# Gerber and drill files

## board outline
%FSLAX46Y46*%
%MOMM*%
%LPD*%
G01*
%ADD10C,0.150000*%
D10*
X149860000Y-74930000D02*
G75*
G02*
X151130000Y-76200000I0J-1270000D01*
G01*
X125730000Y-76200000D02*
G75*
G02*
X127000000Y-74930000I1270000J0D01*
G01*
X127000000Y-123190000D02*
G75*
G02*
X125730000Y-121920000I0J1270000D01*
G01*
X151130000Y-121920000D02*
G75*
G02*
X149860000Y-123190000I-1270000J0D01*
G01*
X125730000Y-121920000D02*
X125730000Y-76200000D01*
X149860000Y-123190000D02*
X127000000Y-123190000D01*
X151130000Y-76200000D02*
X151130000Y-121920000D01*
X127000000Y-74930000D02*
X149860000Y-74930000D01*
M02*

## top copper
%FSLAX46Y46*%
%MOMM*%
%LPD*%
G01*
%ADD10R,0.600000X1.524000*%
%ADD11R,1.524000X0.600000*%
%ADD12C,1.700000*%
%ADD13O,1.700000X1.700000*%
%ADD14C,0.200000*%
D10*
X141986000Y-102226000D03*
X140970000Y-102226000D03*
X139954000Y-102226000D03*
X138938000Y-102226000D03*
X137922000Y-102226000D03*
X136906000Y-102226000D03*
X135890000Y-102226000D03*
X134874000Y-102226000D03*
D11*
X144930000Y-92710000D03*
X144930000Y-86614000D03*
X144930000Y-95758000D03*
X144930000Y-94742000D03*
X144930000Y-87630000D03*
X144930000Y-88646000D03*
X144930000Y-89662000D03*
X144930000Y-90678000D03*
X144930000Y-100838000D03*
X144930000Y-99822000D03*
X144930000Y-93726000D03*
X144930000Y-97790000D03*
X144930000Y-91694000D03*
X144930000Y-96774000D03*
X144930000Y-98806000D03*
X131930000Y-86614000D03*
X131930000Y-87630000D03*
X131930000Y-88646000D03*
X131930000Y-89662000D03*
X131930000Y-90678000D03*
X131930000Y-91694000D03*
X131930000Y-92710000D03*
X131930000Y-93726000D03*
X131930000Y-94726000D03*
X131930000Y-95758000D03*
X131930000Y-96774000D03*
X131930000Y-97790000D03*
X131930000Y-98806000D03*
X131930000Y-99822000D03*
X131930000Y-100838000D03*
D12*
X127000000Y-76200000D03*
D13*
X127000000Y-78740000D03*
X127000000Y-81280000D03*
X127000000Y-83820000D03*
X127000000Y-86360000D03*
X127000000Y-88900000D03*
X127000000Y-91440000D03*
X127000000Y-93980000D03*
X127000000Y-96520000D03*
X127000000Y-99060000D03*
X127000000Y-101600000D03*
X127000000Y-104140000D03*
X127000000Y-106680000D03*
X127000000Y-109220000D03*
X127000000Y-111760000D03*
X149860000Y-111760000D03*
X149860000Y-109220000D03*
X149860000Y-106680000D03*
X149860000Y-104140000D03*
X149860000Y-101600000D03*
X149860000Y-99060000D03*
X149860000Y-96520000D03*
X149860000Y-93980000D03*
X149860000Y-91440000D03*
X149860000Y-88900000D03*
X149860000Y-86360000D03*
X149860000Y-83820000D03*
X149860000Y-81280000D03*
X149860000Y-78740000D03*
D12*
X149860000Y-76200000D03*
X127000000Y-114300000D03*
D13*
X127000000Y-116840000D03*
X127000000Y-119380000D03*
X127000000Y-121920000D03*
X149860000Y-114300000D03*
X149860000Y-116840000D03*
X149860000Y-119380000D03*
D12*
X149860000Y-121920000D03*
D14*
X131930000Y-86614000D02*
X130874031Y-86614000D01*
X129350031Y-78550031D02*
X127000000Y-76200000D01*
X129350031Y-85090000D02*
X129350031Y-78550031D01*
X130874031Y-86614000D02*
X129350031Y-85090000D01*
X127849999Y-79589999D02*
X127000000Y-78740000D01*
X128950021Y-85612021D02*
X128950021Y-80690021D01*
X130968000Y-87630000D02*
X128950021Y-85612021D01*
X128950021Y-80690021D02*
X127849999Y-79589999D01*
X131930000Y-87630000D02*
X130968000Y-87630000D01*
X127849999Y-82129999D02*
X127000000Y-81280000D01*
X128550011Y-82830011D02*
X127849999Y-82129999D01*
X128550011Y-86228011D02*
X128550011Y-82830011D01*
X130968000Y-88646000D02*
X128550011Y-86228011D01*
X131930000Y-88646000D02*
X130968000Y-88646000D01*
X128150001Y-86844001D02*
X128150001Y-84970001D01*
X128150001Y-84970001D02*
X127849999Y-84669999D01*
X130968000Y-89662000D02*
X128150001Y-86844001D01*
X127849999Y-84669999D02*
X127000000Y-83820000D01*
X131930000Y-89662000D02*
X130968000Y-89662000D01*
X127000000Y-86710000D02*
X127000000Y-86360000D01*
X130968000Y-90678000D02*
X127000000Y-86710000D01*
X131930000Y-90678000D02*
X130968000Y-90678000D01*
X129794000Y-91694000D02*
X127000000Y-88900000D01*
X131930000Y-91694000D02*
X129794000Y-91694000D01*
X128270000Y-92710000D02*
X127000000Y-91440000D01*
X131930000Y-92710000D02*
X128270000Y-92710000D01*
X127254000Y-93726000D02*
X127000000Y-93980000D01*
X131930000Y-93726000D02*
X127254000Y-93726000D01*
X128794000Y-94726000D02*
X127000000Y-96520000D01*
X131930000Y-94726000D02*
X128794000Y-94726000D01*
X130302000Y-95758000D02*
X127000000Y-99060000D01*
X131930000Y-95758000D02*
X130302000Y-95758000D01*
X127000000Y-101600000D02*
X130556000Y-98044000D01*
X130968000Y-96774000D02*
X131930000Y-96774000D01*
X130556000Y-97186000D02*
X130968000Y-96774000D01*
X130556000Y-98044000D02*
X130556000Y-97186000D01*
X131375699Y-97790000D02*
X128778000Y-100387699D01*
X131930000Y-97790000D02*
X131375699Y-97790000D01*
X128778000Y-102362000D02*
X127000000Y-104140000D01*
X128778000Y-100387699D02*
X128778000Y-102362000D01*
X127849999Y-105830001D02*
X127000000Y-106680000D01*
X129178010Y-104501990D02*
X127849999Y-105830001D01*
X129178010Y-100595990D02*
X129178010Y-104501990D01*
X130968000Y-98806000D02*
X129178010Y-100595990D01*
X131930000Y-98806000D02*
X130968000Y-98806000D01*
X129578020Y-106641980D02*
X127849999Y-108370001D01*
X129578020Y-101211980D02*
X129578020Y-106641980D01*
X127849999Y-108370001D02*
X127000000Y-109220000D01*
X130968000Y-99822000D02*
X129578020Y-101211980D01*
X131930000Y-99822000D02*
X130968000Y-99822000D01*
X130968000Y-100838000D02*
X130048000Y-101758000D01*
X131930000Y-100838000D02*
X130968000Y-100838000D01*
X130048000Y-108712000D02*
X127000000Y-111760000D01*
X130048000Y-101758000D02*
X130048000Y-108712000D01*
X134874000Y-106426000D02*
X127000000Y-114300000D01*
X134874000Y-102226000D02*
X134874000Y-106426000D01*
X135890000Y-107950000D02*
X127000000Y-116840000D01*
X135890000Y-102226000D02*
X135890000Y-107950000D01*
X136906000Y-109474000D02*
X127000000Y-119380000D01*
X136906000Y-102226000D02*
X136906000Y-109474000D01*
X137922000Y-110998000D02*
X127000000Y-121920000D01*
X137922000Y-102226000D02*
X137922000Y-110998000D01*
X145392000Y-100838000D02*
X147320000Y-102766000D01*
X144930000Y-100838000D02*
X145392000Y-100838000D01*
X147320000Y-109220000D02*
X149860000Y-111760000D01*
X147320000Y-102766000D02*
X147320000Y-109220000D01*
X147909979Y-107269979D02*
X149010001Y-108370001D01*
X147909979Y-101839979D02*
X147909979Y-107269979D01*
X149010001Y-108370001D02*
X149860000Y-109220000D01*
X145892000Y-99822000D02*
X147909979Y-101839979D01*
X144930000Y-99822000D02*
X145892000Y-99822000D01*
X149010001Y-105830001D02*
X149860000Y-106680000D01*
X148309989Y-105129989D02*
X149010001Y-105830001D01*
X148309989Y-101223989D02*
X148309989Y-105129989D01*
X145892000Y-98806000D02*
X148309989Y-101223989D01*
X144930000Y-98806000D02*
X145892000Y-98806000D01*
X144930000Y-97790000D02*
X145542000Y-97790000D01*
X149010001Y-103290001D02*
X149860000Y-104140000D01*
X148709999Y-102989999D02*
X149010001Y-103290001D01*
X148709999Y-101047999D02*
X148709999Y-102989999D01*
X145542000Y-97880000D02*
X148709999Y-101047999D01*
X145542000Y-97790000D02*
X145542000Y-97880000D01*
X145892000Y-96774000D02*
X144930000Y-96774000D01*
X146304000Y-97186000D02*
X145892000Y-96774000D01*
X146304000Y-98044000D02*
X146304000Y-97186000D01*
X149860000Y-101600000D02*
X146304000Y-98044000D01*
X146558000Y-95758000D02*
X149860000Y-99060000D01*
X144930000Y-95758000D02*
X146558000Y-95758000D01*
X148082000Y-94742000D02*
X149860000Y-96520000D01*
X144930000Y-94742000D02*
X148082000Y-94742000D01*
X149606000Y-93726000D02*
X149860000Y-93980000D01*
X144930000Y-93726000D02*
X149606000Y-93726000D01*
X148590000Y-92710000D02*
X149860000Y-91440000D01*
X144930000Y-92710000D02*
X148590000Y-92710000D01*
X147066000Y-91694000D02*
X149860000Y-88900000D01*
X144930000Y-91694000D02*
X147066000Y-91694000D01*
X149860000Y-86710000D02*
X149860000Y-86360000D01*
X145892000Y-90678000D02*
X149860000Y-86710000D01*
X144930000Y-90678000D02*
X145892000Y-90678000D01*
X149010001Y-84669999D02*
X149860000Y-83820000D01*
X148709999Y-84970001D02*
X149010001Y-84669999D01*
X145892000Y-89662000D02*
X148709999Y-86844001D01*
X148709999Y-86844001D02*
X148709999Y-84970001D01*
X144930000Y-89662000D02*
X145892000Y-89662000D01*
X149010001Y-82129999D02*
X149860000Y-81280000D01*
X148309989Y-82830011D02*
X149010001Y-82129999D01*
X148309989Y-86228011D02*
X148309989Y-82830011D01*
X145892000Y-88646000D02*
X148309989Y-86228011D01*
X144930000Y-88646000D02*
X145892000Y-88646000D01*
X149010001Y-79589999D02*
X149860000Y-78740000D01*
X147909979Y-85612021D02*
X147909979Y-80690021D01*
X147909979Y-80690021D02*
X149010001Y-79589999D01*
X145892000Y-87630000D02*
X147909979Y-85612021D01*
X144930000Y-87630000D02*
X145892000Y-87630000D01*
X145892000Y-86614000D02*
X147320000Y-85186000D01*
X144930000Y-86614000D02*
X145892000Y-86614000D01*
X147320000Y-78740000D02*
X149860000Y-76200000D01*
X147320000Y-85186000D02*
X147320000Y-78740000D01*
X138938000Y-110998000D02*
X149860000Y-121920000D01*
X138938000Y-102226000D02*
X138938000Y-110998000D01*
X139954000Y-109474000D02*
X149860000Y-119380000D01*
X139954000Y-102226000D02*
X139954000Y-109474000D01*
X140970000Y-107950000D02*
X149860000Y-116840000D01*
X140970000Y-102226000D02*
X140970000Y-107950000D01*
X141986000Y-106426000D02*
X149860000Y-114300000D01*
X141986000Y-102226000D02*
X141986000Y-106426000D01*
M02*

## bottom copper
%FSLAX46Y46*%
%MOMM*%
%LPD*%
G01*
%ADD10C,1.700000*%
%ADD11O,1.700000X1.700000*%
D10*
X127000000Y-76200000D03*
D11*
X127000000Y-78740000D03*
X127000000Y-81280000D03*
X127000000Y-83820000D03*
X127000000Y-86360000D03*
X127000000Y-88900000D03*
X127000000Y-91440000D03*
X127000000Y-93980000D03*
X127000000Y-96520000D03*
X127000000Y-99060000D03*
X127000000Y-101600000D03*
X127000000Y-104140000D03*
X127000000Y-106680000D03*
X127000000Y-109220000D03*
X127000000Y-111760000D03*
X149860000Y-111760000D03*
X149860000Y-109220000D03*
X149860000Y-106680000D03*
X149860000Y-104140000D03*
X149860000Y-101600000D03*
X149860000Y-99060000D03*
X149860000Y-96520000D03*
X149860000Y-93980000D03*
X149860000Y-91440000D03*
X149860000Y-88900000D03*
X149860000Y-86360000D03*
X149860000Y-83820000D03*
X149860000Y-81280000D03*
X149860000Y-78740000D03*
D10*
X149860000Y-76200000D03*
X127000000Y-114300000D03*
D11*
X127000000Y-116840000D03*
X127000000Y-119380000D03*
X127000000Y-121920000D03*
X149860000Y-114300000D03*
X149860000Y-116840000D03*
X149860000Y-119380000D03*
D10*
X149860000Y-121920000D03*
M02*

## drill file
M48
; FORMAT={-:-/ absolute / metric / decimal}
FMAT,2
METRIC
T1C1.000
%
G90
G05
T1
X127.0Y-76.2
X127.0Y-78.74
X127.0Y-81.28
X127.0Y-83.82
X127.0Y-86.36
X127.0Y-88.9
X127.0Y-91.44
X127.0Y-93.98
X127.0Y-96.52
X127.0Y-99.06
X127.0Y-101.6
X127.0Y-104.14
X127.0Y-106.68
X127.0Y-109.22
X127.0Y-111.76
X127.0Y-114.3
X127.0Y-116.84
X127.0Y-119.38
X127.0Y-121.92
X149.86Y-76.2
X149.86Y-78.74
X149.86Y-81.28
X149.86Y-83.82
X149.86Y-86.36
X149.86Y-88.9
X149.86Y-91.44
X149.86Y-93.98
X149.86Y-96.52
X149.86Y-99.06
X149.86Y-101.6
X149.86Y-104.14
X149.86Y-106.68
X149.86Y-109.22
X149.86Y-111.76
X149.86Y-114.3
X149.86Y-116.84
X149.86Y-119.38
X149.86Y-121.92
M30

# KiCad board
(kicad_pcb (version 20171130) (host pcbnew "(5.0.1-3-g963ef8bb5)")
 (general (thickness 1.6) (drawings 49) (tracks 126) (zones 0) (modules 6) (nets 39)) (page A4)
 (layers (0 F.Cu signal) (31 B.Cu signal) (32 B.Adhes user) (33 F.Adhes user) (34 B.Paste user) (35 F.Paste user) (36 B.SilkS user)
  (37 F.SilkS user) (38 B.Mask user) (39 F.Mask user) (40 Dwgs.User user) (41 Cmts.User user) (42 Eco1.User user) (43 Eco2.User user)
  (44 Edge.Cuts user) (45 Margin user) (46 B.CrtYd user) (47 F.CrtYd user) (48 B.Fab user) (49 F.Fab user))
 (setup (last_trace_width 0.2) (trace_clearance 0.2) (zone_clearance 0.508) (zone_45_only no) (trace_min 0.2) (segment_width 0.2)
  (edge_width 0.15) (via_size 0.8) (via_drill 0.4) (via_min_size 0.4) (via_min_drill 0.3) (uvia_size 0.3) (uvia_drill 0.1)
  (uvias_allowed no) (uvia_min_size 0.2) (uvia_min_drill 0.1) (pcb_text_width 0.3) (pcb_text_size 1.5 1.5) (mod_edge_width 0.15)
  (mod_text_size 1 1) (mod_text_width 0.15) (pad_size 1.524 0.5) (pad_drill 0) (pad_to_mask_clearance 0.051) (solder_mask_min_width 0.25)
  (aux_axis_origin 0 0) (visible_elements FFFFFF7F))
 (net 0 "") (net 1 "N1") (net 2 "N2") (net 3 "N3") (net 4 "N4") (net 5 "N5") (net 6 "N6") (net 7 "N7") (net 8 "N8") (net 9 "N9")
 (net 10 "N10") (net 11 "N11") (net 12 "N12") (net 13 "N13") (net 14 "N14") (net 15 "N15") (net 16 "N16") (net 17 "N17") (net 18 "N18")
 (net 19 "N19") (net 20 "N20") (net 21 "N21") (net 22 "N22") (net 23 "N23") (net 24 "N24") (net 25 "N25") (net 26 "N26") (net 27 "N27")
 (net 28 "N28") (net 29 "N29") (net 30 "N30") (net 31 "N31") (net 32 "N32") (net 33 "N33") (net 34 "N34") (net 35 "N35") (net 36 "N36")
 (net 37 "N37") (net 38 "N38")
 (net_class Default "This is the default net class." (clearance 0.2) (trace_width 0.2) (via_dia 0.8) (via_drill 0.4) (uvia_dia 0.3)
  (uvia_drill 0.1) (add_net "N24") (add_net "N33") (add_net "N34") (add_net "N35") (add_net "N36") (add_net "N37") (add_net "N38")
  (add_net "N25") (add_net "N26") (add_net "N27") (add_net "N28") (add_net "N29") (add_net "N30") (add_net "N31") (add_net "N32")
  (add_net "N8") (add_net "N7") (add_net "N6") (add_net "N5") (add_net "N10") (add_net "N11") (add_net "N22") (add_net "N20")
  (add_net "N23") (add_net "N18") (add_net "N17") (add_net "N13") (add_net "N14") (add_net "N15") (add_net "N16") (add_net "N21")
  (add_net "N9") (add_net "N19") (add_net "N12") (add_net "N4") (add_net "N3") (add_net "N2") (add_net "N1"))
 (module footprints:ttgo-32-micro (layer F.Cu) (at 138.43 93.726)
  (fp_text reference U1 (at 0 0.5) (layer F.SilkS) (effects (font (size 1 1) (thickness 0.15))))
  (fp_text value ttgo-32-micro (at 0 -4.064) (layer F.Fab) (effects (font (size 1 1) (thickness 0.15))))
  (pad 23 smd rect (at 3.556 8.5 90) (size 1.524 0.6) (layers F.Cu F.Paste F.Mask) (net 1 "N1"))
  (pad 22 smd rect (at 2.54 8.5 90) (size 1.524 0.6) (layers F.Cu F.Paste F.Mask) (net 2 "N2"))
  (pad 21 smd rect (at 1.524 8.5 90) (size 1.524 0.6) (layers F.Cu F.Paste F.Mask) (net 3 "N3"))
  (pad 20 smd rect (at 0.508 8.5 90) (size 1.524 0.6) (layers F.Cu F.Paste F.Mask) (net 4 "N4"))
  (pad 19 smd rect (at -0.508 8.5 90) (size 1.524 0.6) (layers F.Cu F.Paste F.Mask) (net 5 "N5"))
  (pad 18 smd rect (at -1.524 8.5 90) (size 1.524 0.6) (layers F.Cu F.Paste F.Mask) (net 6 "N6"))
  (pad 17 smd rect (at -2.54 8.5 90) (size 1.524 0.6) (layers F.Cu F.Paste F.Mask) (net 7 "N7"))
  (pad 16 smd rect (at -3.556 8.5 90) (size 1.524 0.6) (layers F.Cu F.Paste F.Mask) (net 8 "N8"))
  (pad 32 smd rect (at 6.5 -1.016) (size 1.524 0.6) (layers F.Cu F.Paste F.Mask) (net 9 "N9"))
  (pad 38 smd rect (at 6.5 -7.112) (size 1.524 0.6) (layers F.Cu F.Paste F.Mask) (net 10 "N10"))
  (pad 29 smd rect (at 6.5 2.032) (size 1.524 0.6) (layers F.Cu F.Paste F.Mask) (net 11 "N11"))
  (pad 30 smd rect (at 6.5 1.016) (size 1.524 0.6) (layers F.Cu F.Paste F.Mask) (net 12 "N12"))
  (pad 37 smd rect (at 6.5 -6.096) (size 1.524 0.6) (layers F.Cu F.Paste F.Mask) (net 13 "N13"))
  (pad 36 smd rect (at 6.5 -5.08) (size 1.524 0.6) (layers F.Cu F.Paste F.Mask) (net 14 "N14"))
  (pad 35 smd rect (at 6.5 -4.064) (size 1.524 0.6) (layers F.Cu F.Paste F.Mask) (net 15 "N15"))
  (pad 34 smd rect (at 6.5 -3.048) (size 1.524 0.6) (layers F.Cu F.Paste F.Mask) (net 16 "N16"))
  (pad 24 smd rect (at 6.5 7.112) (size 1.524 0.6) (layers F.Cu F.Paste F.Mask) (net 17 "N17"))
  (pad 25 smd rect (at 6.5 6.096) (size 1.524 0.6) (layers F.Cu F.Paste F.Mask) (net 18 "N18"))
  (pad 31 smd rect (at 6.5 0) (size 1.524 0.6) (layers F.Cu F.Paste F.Mask) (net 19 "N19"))
  (pad 27 smd rect (at 6.5 4.064) (size 1.524 0.6) (layers F.Cu F.Paste F.Mask) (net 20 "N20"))
  (pad 33 smd rect (at 6.5 -2.032) (size 1.524 0.6) (layers F.Cu F.Paste F.Mask) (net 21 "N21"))
  (pad 28 smd rect (at 6.5 3.048) (size 1.524 0.6) (layers F.Cu F.Paste F.Mask) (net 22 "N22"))
  (pad 26 smd rect (at 6.5 5.08) (size 1.524 0.6) (layers F.Cu F.Paste F.Mask) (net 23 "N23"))
  (pad 1 smd rect (at -6.5 -7.112) (size 1.524 0.6) (layers F.Cu F.Paste F.Mask) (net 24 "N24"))
  (pad 2 smd rect (at -6.5 -6.096) (size 1.524 0.6) (layers F.Cu F.Paste F.Mask) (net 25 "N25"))
  (pad 3 smd rect (at -6.5 -5.08) (size 1.524 0.6) (layers F.Cu F.Paste F.Mask) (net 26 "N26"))
  (pad 4 smd rect (at -6.5 -4.064) (size 1.524 0.6) (layers F.Cu F.Paste F.Mask) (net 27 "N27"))
  (pad 5 smd rect (at -6.5 -3.048) (size 1.524 0.6) (layers F.Cu F.Paste F.Mask) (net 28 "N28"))
  (pad 6 smd rect (at -6.5 -2.032) (size 1.524 0.6) (layers F.Cu F.Paste F.Mask) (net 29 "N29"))
  (pad 7 smd rect (at -6.5 -1.016) (size 1.524 0.6) (layers F.Cu F.Paste F.Mask) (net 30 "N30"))
  (pad 8 smd rect (at -6.5 0) (size 1.524 0.6) (layers F.Cu F.Paste F.Mask) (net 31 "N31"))
  (pad 9 smd rect (at -6.5 1) (size 1.524 0.6) (layers F.Cu F.Paste F.Mask) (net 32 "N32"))
  (pad 10 smd rect (at -6.5 2.032) (size 1.524 0.6) (layers F.Cu F.Paste F.Mask) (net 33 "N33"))
  (pad 11 smd rect (at -6.5 3.048) (size 1.524 0.6) (layers F.Cu F.Paste F.Mask) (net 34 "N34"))
  (pad 12 smd rect (at -6.5 4.064) (size 1.524 0.6) (layers F.Cu F.Paste F.Mask) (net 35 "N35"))
  (pad 13 smd rect (at -6.5 5.08) (size 1.524 0.6) (layers F.Cu F.Paste F.Mask) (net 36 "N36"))
  (pad 14 smd rect (at -6.5 6.096) (size 1.524 0.6) (layers F.Cu F.Paste F.Mask) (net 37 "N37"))
  (pad 15 smd rect (at -6.5 7.112) (size 1.524 0.6) (layers F.Cu F.Paste F.Mask) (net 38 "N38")))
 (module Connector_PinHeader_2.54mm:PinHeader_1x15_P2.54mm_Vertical (layer B.Cu) (at 127 76.2 180)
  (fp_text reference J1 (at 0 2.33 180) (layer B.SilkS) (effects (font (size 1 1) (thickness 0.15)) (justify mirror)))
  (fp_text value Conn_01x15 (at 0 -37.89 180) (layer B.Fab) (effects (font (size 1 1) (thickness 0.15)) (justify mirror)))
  (pad 1 thru_hole circle (at 0 0 180) (size 1.7 1.7) (drill 1) (layers *.Cu *.Mask) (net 24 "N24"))
  (pad 2 thru_hole oval (at 0 -2.54 180) (size 1.7 1.7) (drill 1) (layers *.Cu *.Mask) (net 25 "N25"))
  (pad 3 thru_hole oval (at 0 -5.08 180) (size 1.7 1.7) (drill 1) (layers *.Cu *.Mask) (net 26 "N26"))
  (pad 4 thru_hole oval (at 0 -7.62 180) (size 1.7 1.7) (drill 1) (layers *.Cu *.Mask) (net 27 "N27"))
  (pad 5 thru_hole oval (at 0 -10.16 180) (size 1.7 1.7) (drill 1) (layers *.Cu *.Mask) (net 28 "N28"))
  (pad 6 thru_hole oval (at 0 -12.7 180) (size 1.7 1.7) (drill 1) (layers *.Cu *.Mask) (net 29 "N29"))
  (pad 7 thru_hole oval (at 0 -15.24 180) (size 1.7 1.7) (drill 1) (layers *.Cu *.Mask) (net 30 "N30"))
  (pad 8 thru_hole oval (at 0 -17.78 180) (size 1.7 1.7) (drill 1) (layers *.Cu *.Mask) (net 31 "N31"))
  (pad 9 thru_hole oval (at 0 -20.32 180) (size 1.7 1.7) (drill 1) (layers *.Cu *.Mask) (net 32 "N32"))
  (pad 10 thru_hole oval (at 0 -22.86 180) (size 1.7 1.7) (drill 1) (layers *.Cu *.Mask) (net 33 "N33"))
  (pad 11 thru_hole oval (at 0 -25.4 180) (size 1.7 1.7) (drill 1) (layers *.Cu *.Mask) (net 34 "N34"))
  (pad 12 thru_hole oval (at 0 -27.94 180) (size 1.7 1.7) (drill 1) (layers *.Cu *.Mask) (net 35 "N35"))
  (pad 13 thru_hole oval (at 0 -30.48 180) (size 1.7 1.7) (drill 1) (layers *.Cu *.Mask) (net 36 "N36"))
  (pad 14 thru_hole oval (at 0 -33.02 180) (size 1.7 1.7) (drill 1) (layers *.Cu *.Mask) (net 37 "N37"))
  (pad 15 thru_hole oval (at 0 -35.56 180) (size 1.7 1.7) (drill 1) (layers *.Cu *.Mask) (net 38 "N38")))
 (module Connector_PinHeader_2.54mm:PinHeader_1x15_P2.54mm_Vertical (layer B.Cu) (at 149.86 76.2 180)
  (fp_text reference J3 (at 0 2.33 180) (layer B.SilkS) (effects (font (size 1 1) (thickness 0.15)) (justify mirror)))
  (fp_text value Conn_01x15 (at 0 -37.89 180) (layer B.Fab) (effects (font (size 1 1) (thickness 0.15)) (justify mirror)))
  (pad 15 thru_hole oval (at 0 -35.56 180) (size 1.7 1.7) (drill 1) (layers *.Cu *.Mask) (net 17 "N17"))
  (pad 14 thru_hole oval (at 0 -33.02 180) (size 1.7 1.7) (drill 1) (layers *.Cu *.Mask) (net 18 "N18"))
  (pad 13 thru_hole oval (at 0 -30.48 180) (size 1.7 1.7) (drill 1) (layers *.Cu *.Mask) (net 23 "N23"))
  (pad 12 thru_hole oval (at 0 -27.94 180) (size 1.7 1.7) (drill 1) (layers *.Cu *.Mask) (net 20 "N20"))
  (pad 11 thru_hole oval (at 0 -25.4 180) (size 1.7 1.7) (drill 1) (layers *.Cu *.Mask) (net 22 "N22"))
  (pad 10 thru_hole oval (at 0 -22.86 180) (size 1.7 1.7) (drill 1) (layers *.Cu *.Mask) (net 11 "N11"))
  (pad 9 thru_hole oval (at 0 -20.32 180) (size 1.7 1.7) (drill 1) (layers *.Cu *.Mask) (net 12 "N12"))
  (pad 8 thru_hole oval (at 0 -17.78 180) (size 1.7 1.7) (drill 1) (layers *.Cu *.Mask) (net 19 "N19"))
  (pad 7 thru_hole oval (at 0 -15.24 180) (size 1.7 1.7) (drill 1) (layers *.Cu *.Mask) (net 9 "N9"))
  (pad 6 thru_hole oval (at 0 -12.7 180) (size 1.7 1.7) (drill 1) (layers *.Cu *.Mask) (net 21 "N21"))
  (pad 5 thru_hole oval (at 0 -10.16 180) (size 1.7 1.7) (drill 1) (layers *.Cu *.Mask) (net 16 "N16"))
  (pad 4 thru_hole oval (at 0 -7.62 180) (size 1.7 1.7) (drill 1) (layers *.Cu *.Mask) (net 15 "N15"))
  (pad 3 thru_hole oval (at 0 -5.08 180) (size 1.7 1.7) (drill 1) (layers *.Cu *.Mask) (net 14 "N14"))
  (pad 2 thru_hole oval (at 0 -2.54 180) (size 1.7 1.7) (drill 1) (layers *.Cu *.Mask) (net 13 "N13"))
  (pad 1 thru_hole circle (at 0 0 180) (size 1.7 1.7) (drill 1) (layers *.Cu *.Mask) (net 10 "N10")))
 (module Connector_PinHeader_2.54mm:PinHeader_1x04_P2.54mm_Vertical (layer B.Cu) (at 127 114.3 180)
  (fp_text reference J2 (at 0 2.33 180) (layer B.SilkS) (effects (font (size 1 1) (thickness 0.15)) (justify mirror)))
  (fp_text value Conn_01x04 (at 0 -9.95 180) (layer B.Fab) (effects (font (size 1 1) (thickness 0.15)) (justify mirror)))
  (pad 1 thru_hole circle (at 0 0 180) (size 1.7 1.7) (drill 1) (layers *.Cu *.Mask) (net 8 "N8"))
  (pad 2 thru_hole oval (at 0 -2.54 180) (size 1.7 1.7) (drill 1) (layers *.Cu *.Mask) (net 7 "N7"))
  (pad 3 thru_hole oval (at 0 -5.08 180) (size 1.7 1.7) (drill 1) (layers *.Cu *.Mask) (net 6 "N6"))
  (pad 4 thru_hole oval (at 0 -7.62 180) (size 1.7 1.7) (drill 1) (layers *.Cu *.Mask) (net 5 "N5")))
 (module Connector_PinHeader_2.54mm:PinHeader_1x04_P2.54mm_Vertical (layer B.Cu) (at 149.86 121.92)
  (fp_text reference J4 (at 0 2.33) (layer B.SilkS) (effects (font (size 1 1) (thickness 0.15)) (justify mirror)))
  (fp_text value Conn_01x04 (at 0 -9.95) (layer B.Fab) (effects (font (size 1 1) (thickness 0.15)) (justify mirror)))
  (pad 4 thru_hole oval (at 0 -7.62) (size 1.7 1.7) (drill 1) (layers *.Cu *.Mask) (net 1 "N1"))
  (pad 3 thru_hole oval (at 0 -5.08) (size 1.7 1.7) (drill 1) (layers *.Cu *.Mask) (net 2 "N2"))
  (pad 2 thru_hole oval (at 0 -2.54) (size 1.7 1.7) (drill 1) (layers *.Cu *.Mask) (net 3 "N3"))
  (pad 1 thru_hole circle (at 0 0) (size 1.7 1.7) (drill 1) (layers *.Cu *.Mask) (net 4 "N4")))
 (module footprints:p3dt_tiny (layer F.Cu) (at 138.43 110.49)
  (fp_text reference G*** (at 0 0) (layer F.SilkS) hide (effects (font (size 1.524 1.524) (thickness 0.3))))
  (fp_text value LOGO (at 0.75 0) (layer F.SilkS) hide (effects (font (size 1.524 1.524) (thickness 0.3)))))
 (gr_arc (start 149.86 76.2) (end 151.13 76.2) (angle -90) (layer Edge.Cuts) (width 0.15))
 (gr_arc (start 127 76.2) (end 127 74.93) (angle -90) (layer Edge.Cuts) (width 0.15))
 (gr_arc (start 127 121.92) (end 125.73 121.92) (angle -90) (layer Edge.Cuts) (width 0.15))
 (gr_arc (start 149.86 121.92) (end 149.86 123.19) (angle -90) (layer Edge.Cuts) (width 0.15))
 (gr_line (start 125.73 121.92) (end 125.73 76.2) (layer Edge.Cuts) (width 0.15))
 (gr_line (start 149.86 123.19) (end 127 123.19) (layer Edge.Cuts) (width 0.15))
 (gr_line (start 151.13 76.2) (end 151.13 121.92) (layer Edge.Cuts) (width 0.15))
 (gr_line (start 127 74.93) (end 149.86 74.93) (layer Edge.Cuts) (width 0.15))
 (segment (start 131.93 86.614) (end 130.874031 86.614) (width 0.2) (layer F.Cu) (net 24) (status 10))
 (segment (start 129.350031 78.550031) (end 127 76.2) (width 0.2) (layer F.Cu) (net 24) (status 20))
 (segment (start 129.350031 85.09) (end 129.350031 78.550031) (width 0.2) (layer F.Cu) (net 24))
 (segment (start 130.874031 86.614) (end 129.350031 85.09) (width 0.2) (layer F.Cu) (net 24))
 (segment (start 127.849999 79.589999) (end 127 78.74) (width 0.2) (layer F.Cu) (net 25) (status 30))
 (segment (start 128.950021 85.612021) (end 128.950021 80.690021) (width 0.2) (layer F.Cu) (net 25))
 (segment (start 130.968 87.63) (end 128.950021 85.612021) (width 0.2) (layer F.Cu) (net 25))
 (segment (start 128.950021 80.690021) (end 127.849999 79.589999) (width 0.2) (layer F.Cu) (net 25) (status 20))
 (segment (start 131.93 87.63) (end 130.968 87.63) (width 0.2) (layer F.Cu) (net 25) (status 10))
 (segment (start 127.849999 82.129999) (end 127 81.28) (width 0.2) (layer F.Cu) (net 26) (status 30))
 (segment (start 128.550011 82.830011) (end 127.849999 82.129999) (width 0.2) (layer F.Cu) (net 26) (status 20))
 (segment (start 128.550011 86.228011) (end 128.550011 82.830011) (width 0.2) (layer F.Cu) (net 26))
 (segment (start 130.968 88.646) (end 128.550011 86.228011) (width 0.2) (layer F.Cu) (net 26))
 (segment (start 131.93 88.646) (end 130.968 88.646) (width 0.2) (layer F.Cu) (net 26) (status 10))
 (segment (start 128.150001 86.844001) (end 128.150001 84.970001) (width 0.2) (layer F.Cu) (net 27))
 (segment (start 128.150001 84.970001) (end 127.849999 84.669999) (width 0.2) (layer F.Cu) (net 27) (status 20))
 (segment (start 130.968 89.662) (end 128.150001 86.844001) (width 0.2) (layer F.Cu) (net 27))
 (segment (start 127.849999 84.669999) (end 127 83.82) (width 0.2) (layer F.Cu) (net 27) (status 30))
 (segment (start 131.93 89.662) (end 130.968 89.662) (width 0.2) (layer F.Cu) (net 27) (status 10))
 (segment (start 127 86.71) (end 127 86.36) (width 0.2) (layer F.Cu) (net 28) (status 30))
 (segment (start 130.968 90.678) (end 127 86.71) (width 0.2) (layer F.Cu) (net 28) (status 20))
 (segment (start 131.93 90.678) (end 130.968 90.678) (width 0.2) (layer F.Cu) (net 28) (status 10))
 (segment (start 129.794 91.694) (end 127 88.9) (width 0.2) (layer F.Cu) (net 29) (status 20))
 (segment (start 131.93 91.694) (end 129.794 91.694) (width 0.2) (layer F.Cu) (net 29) (status 10))
 (segment (start 128.27 92.71) (end 127 91.44) (width 0.2) (layer F.Cu) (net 30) (status 20))
 (segment (start 131.93 92.71) (end 128.27 92.71) (width 0.2) (layer F.Cu) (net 30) (status 10))
 (segment (start 127.254 93.726) (end 127 93.98) (width 0.2) (layer F.Cu) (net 31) (status 30))
 (segment (start 131.93 93.726) (end 127.254 93.726) (width 0.2) (layer F.Cu) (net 31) (status 30))
 (segment (start 128.794 94.726) (end 127 96.52) (width 0.2) (layer F.Cu) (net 32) (status 20))
 (segment (start 131.93 94.726) (end 128.794 94.726) (width 0.2) (layer F.Cu) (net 32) (status 10))
 (segment (start 130.302 95.758) (end 127 99.06) (width 0.2) (layer F.Cu) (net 33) (status 20))
 (segment (start 131.93 95.758) (end 130.302 95.758) (width 0.2) (layer F.Cu) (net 33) (status 10))
 (segment (start 127 101.6) (end 130.556 98.044) (width 0.2) (layer F.Cu) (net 34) (status 10))
 (segment (start 130.968 96.774) (end 131.93 96.774) (width 0.2) (layer F.Cu) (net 34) (status 20))
 (segment (start 130.556 97.186) (end 130.968 96.774) (width 0.2) (layer F.Cu) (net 34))
 (segment (start 130.556 98.044) (end 130.556 97.186) (width 0.2) (layer F.Cu) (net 34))
 (segment (start 131.375699 97.79) (end 128.778 100.387699) (width 0.2) (layer F.Cu) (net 35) (status 10))
 (segment (start 131.93 97.79) (end 131.375699 97.79) (width 0.2) (layer F.Cu) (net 35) (status 30))
 (segment (start 128.778 102.362) (end 127 104.14) (width 0.2) (layer F.Cu) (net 35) (status 20))
 (segment (start 128.778 100.387699) (end 128.778 102.362) (width 0.2) (layer F.Cu) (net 35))
 (segment (start 127.849999 105.830001) (end 127 106.68) (width 0.2) (layer F.Cu) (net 36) (status 30))
 (segment (start 129.17801 104.50199) (end 127.849999 105.830001) (width 0.2) (layer F.Cu) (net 36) (status 20))
 (segment (start 129.17801 100.59599) (end 129.17801 104.50199) (width 0.2) (layer F.Cu) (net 36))
 (segment (start 130.968 98.806) (end 129.17801 100.59599) (width 0.2) (layer F.Cu) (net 36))
 (segment (start 131.93 98.806) (end 130.968 98.806) (width 0.2) (layer F.Cu) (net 36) (status 10))
 (segment (start 129.57802 106.64198) (end 127.849999 108.370001) (width 0.2) (layer F.Cu) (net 37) (status 20))
 (segment (start 129.57802 101.21198) (end 129.57802 106.64198) (width 0.2) (layer F.Cu) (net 37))
 (segment (start 127.849999 108.370001) (end 127 109.22) (width 0.2) (layer F.Cu) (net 37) (status 30))
 (segment (start 130.968 99.822) (end 129.57802 101.21198) (width 0.2) (layer F.Cu) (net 37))
 (segment (start 131.93 99.822) (end 130.968 99.822) (width 0.2) (layer F.Cu) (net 37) (status 10))
 (segment (start 130.968 100.838) (end 130.048 101.758) (width 0.2) (layer F.Cu) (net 38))
 (segment (start 131.93 100.838) (end 130.968 100.838) (width 0.2) (layer F.Cu) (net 38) (status 10))
 (segment (start 130.048 108.712) (end 127 111.76) (width 0.2) (layer F.Cu) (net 38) (status 20))
 (segment (start 130.048 101.758) (end 130.048 108.712) (width 0.2) (layer F.Cu) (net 38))
 (segment (start 134.874 106.426) (end 127 114.3) (width 0.2) (layer F.Cu) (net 8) (status 20))
 (segment (start 134.874 102.226) (end 134.874 106.426) (width 0.2) (layer F.Cu) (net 8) (status 10))
 (segment (start 135.89 107.95) (end 127 116.84) (width 0.2) (layer F.Cu) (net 7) (status 20))
 (segment (start 135.89 102.226) (end 135.89 107.95) (width 0.2) (layer F.Cu) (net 7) (status 10))
 (segment (start 136.906 109.474) (end 127 119.38) (width 0.2) (layer F.Cu) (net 6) (status 20))
 (segment (start 136.906 102.226) (end 136.906 109.474) (width 0.2) (layer F.Cu) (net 6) (status 10))
 (segment (start 137.922 110.998) (end 127 121.92) (width 0.2) (layer F.Cu) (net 5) (status 20))
 (segment (start 137.922 102.226) (end 137.922 110.998) (width 0.2) (layer F.Cu) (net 5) (status 10))
 (segment (start 145.392 100.838) (end 147.32 102.766) (width 0.2) (layer F.Cu) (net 17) (status 10))
 (segment (start 144.93 100.838) (end 145.392 100.838) (width 0.2) (layer F.Cu) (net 17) (status 30))
 (segment (start 147.32 109.22) (end 149.86 111.76) (width 0.2) (layer F.Cu) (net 17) (status 20))
 (segment (start 147.32 102.766) (end 147.32 109.22) (width 0.2) (layer F.Cu) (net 17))
 (segment (start 147.909979 107.269979) (end 149.010001 108.370001) (width 0.2) (layer F.Cu) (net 18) (status 20))
 (segment (start 147.909979 101.839979) (end 147.909979 107.269979) (width 0.2) (layer F.Cu) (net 18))
 (segment (start 149.010001 108.370001) (end 149.86 109.22) (width 0.2) (layer F.Cu) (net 18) (status 30))
 (segment (start 145.892 99.822) (end 147.909979 101.839979) (width 0.2) (layer F.Cu) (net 18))
 (segment (start 144.93 99.822) (end 145.892 99.822) (width 0.2) (layer F.Cu) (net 18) (status 10))
 (segment (start 149.010001 105.830001) (end 149.86 106.68) (width 0.2) (layer F.Cu) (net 23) (status 30))
 (segment (start 148.309989 105.129989) (end 149.010001 105.830001) (width 0.2) (layer F.Cu) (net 23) (status 20))
 (segment (start 148.309989 101.223989) (end 148.309989 105.129989) (width 0.2) (layer F.Cu) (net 23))
 (segment (start 145.892 98.806) (end 148.309989 101.223989) (width 0.2) (layer F.Cu) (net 23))
 (segment (start 144.93 98.806) (end 145.892 98.806) (width 0.2) (layer F.Cu) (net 23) (status 10))
 (segment (start 144.93 97.79) (end 145.542 97.79) (width 0.2) (layer F.Cu) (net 20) (status 30))
 (segment (start 149.010001 103.290001) (end 149.86 104.14) (width 0.2) (layer F.Cu) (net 20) (status 30))
 (segment (start 148.709999 102.989999) (end 149.010001 103.290001) (width 0.2) (layer F.Cu) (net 20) (status 20))
 (segment (start 148.709999 101.047999) (end 148.709999 102.989999) (width 0.2) (layer F.Cu) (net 20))
 (segment (start 145.542 97.88) (end 148.709999 101.047999) (width 0.2) (layer F.Cu) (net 20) (status 10))
 (segment (start 145.542 97.79) (end 145.542 97.88) (width 0.2) (layer F.Cu) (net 20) (status 30))
 (segment (start 145.892 96.774) (end 144.93 96.774) (width 0.2) (layer F.Cu) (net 22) (status 20))
 (segment (start 146.304 97.186) (end 145.892 96.774) (width 0.2) (layer F.Cu) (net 22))
 (segment (start 146.304 98.044) (end 146.304 97.186) (width 0.2) (layer F.Cu) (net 22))
 (segment (start 149.86 101.6) (end 146.304 98.044) (width 0.2) (layer F.Cu) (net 22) (status 10))
 (segment (start 146.558 95.758) (end 149.86 99.06) (width 0.2) (layer F.Cu) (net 11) (status 20))
 (segment (start 144.93 95.758) (end 146.558 95.758) (width 0.2) (layer F.Cu) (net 11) (status 10))
 (segment (start 148.082 94.742) (end 149.86 96.52) (width 0.2) (layer F.Cu) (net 12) (status 20))
 (segment (start 144.93 94.742) (end 148.082 94.742) (width 0.2) (layer F.Cu) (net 12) (status 10))
 (segment (start 149.606 93.726) (end 149.86 93.98) (width 0.2) (layer F.Cu) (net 19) (status 30))
 (segment (start 144.93 93.726) (end 149.606 93.726) (width 0.2) (layer F.Cu) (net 19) (status 30))
 (segment (start 148.59 92.71) (end 149.86 91.44) (width 0.2) (layer F.Cu) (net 9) (status 20))
 (segment (start 144.93 92.71) (end 148.59 92.71) (width 0.2) (layer F.Cu) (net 9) (status 10))
 (segment (start 147.066 91.694) (end 149.86 88.9) (width 0.2) (layer F.Cu) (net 21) (status 20))
 (segment (start 144.93 91.694) (end 147.066 91.694) (width 0.2) (layer F.Cu) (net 21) (status 10))
 (segment (start 149.86 86.71) (end 149.86 86.36) (width 0.2) (layer F.Cu) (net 16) (status 30))
 (segment (start 145.892 90.678) (end 149.86 86.71) (width 0.2) (layer F.Cu) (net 16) (status 20))
 (segment (start 144.93 90.678) (end 145.892 90.678) (width 0.2) (layer F.Cu) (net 16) (status 10))
 (segment (start 149.010001 84.669999) (end 149.86 83.82) (width 0.2) (layer F.Cu) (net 15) (status 30))
 (segment (start 148.709999 84.970001) (end 149.010001 84.669999) (width 0.2) (layer F.Cu) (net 15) (status 20))
 (segment (start 145.892 89.662) (end 148.709999 86.844001) (width 0.2) (layer F.Cu) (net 15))
 (segment (start 148.709999 86.844001) (end 148.709999 84.970001) (width 0.2) (layer F.Cu) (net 15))
 (segment (start 144.93 89.662) (end 145.892 89.662) (width 0.2) (layer F.Cu) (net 15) (status 10))
 (segment (start 149.010001 82.129999) (end 149.86 81.28) (width 0.2) (layer F.Cu) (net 14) (status 30))
 (segment (start 148.309989 82.830011) (end 149.010001 82.129999) (width 0.2) (layer F.Cu) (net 14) (status 20))
 (segment (start 148.309989 86.228011) (end 148.309989 82.830011) (width 0.2) (layer F.Cu) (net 14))
 (segment (start 145.892 88.646) (end 148.309989 86.228011) (width 0.2) (layer F.Cu) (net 14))
 (segment (start 144.93 88.646) (end 145.892 88.646) (width 0.2) (layer F.Cu) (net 14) (status 10))
 (segment (start 149.010001 79.589999) (end 149.86 78.74) (width 0.2) (layer F.Cu) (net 13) (status 30))
 (segment (start 147.909979 85.612021) (end 147.909979 80.690021) (width 0.2) (layer F.Cu) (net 13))
 (segment (start 147.909979 80.690021) (end 149.010001 79.589999) (width 0.2) (layer F.Cu) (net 13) (status 20))
 (segment (start 145.892 87.63) (end 147.909979 85.612021) (width 0.2) (layer F.Cu) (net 13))
 (segment (start 144.93 87.63) (end 145.892 87.63) (width 0.2) (layer F.Cu) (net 13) (status 10))
 (segment (start 145.892 86.614) (end 147.32 85.186) (width 0.2) (layer F.Cu) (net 10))
 (segment (start 144.93 86.614) (end 145.892 86.614) (width 0.2) (layer F.Cu) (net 10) (status 10))
 (segment (start 147.32 78.74) (end 149.86 76.2) (width 0.2) (layer F.Cu) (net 10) (status 20))
 (segment (start 147.32 85.186) (end 147.32 78.74) (width 0.2) (layer F.Cu) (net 10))
 (segment (start 138.938 110.998) (end 149.86 121.92) (width 0.2) (layer F.Cu) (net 4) (status 20))
 (segment (start 138.938 102.226) (end 138.938 110.998) (width 0.2) (layer F.Cu) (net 4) (status 10))
 (segment (start 139.954 109.474) (end 149.86 119.38) (width 0.2) (layer F.Cu) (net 3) (status 20))
 (segment (start 139.954 102.226) (end 139.954 109.474) (width 0.2) (layer F.Cu) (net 3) (status 10))
 (segment (start 140.97 107.95) (end 149.86 116.84) (width 0.2) (layer F.Cu) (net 2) (status 20))
 (segment (start 140.97 102.226) (end 140.97 107.95) (width 0.2) (layer F.Cu) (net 2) (status 10))
 (segment (start 141.986 106.426) (end 149.86 114.3) (width 0.2) (layer F.Cu) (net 1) (status 20))
 (segment (start 141.986 102.226) (end 141.986 106.426) (width 0.2) (layer F.Cu) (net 1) (status 10)))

